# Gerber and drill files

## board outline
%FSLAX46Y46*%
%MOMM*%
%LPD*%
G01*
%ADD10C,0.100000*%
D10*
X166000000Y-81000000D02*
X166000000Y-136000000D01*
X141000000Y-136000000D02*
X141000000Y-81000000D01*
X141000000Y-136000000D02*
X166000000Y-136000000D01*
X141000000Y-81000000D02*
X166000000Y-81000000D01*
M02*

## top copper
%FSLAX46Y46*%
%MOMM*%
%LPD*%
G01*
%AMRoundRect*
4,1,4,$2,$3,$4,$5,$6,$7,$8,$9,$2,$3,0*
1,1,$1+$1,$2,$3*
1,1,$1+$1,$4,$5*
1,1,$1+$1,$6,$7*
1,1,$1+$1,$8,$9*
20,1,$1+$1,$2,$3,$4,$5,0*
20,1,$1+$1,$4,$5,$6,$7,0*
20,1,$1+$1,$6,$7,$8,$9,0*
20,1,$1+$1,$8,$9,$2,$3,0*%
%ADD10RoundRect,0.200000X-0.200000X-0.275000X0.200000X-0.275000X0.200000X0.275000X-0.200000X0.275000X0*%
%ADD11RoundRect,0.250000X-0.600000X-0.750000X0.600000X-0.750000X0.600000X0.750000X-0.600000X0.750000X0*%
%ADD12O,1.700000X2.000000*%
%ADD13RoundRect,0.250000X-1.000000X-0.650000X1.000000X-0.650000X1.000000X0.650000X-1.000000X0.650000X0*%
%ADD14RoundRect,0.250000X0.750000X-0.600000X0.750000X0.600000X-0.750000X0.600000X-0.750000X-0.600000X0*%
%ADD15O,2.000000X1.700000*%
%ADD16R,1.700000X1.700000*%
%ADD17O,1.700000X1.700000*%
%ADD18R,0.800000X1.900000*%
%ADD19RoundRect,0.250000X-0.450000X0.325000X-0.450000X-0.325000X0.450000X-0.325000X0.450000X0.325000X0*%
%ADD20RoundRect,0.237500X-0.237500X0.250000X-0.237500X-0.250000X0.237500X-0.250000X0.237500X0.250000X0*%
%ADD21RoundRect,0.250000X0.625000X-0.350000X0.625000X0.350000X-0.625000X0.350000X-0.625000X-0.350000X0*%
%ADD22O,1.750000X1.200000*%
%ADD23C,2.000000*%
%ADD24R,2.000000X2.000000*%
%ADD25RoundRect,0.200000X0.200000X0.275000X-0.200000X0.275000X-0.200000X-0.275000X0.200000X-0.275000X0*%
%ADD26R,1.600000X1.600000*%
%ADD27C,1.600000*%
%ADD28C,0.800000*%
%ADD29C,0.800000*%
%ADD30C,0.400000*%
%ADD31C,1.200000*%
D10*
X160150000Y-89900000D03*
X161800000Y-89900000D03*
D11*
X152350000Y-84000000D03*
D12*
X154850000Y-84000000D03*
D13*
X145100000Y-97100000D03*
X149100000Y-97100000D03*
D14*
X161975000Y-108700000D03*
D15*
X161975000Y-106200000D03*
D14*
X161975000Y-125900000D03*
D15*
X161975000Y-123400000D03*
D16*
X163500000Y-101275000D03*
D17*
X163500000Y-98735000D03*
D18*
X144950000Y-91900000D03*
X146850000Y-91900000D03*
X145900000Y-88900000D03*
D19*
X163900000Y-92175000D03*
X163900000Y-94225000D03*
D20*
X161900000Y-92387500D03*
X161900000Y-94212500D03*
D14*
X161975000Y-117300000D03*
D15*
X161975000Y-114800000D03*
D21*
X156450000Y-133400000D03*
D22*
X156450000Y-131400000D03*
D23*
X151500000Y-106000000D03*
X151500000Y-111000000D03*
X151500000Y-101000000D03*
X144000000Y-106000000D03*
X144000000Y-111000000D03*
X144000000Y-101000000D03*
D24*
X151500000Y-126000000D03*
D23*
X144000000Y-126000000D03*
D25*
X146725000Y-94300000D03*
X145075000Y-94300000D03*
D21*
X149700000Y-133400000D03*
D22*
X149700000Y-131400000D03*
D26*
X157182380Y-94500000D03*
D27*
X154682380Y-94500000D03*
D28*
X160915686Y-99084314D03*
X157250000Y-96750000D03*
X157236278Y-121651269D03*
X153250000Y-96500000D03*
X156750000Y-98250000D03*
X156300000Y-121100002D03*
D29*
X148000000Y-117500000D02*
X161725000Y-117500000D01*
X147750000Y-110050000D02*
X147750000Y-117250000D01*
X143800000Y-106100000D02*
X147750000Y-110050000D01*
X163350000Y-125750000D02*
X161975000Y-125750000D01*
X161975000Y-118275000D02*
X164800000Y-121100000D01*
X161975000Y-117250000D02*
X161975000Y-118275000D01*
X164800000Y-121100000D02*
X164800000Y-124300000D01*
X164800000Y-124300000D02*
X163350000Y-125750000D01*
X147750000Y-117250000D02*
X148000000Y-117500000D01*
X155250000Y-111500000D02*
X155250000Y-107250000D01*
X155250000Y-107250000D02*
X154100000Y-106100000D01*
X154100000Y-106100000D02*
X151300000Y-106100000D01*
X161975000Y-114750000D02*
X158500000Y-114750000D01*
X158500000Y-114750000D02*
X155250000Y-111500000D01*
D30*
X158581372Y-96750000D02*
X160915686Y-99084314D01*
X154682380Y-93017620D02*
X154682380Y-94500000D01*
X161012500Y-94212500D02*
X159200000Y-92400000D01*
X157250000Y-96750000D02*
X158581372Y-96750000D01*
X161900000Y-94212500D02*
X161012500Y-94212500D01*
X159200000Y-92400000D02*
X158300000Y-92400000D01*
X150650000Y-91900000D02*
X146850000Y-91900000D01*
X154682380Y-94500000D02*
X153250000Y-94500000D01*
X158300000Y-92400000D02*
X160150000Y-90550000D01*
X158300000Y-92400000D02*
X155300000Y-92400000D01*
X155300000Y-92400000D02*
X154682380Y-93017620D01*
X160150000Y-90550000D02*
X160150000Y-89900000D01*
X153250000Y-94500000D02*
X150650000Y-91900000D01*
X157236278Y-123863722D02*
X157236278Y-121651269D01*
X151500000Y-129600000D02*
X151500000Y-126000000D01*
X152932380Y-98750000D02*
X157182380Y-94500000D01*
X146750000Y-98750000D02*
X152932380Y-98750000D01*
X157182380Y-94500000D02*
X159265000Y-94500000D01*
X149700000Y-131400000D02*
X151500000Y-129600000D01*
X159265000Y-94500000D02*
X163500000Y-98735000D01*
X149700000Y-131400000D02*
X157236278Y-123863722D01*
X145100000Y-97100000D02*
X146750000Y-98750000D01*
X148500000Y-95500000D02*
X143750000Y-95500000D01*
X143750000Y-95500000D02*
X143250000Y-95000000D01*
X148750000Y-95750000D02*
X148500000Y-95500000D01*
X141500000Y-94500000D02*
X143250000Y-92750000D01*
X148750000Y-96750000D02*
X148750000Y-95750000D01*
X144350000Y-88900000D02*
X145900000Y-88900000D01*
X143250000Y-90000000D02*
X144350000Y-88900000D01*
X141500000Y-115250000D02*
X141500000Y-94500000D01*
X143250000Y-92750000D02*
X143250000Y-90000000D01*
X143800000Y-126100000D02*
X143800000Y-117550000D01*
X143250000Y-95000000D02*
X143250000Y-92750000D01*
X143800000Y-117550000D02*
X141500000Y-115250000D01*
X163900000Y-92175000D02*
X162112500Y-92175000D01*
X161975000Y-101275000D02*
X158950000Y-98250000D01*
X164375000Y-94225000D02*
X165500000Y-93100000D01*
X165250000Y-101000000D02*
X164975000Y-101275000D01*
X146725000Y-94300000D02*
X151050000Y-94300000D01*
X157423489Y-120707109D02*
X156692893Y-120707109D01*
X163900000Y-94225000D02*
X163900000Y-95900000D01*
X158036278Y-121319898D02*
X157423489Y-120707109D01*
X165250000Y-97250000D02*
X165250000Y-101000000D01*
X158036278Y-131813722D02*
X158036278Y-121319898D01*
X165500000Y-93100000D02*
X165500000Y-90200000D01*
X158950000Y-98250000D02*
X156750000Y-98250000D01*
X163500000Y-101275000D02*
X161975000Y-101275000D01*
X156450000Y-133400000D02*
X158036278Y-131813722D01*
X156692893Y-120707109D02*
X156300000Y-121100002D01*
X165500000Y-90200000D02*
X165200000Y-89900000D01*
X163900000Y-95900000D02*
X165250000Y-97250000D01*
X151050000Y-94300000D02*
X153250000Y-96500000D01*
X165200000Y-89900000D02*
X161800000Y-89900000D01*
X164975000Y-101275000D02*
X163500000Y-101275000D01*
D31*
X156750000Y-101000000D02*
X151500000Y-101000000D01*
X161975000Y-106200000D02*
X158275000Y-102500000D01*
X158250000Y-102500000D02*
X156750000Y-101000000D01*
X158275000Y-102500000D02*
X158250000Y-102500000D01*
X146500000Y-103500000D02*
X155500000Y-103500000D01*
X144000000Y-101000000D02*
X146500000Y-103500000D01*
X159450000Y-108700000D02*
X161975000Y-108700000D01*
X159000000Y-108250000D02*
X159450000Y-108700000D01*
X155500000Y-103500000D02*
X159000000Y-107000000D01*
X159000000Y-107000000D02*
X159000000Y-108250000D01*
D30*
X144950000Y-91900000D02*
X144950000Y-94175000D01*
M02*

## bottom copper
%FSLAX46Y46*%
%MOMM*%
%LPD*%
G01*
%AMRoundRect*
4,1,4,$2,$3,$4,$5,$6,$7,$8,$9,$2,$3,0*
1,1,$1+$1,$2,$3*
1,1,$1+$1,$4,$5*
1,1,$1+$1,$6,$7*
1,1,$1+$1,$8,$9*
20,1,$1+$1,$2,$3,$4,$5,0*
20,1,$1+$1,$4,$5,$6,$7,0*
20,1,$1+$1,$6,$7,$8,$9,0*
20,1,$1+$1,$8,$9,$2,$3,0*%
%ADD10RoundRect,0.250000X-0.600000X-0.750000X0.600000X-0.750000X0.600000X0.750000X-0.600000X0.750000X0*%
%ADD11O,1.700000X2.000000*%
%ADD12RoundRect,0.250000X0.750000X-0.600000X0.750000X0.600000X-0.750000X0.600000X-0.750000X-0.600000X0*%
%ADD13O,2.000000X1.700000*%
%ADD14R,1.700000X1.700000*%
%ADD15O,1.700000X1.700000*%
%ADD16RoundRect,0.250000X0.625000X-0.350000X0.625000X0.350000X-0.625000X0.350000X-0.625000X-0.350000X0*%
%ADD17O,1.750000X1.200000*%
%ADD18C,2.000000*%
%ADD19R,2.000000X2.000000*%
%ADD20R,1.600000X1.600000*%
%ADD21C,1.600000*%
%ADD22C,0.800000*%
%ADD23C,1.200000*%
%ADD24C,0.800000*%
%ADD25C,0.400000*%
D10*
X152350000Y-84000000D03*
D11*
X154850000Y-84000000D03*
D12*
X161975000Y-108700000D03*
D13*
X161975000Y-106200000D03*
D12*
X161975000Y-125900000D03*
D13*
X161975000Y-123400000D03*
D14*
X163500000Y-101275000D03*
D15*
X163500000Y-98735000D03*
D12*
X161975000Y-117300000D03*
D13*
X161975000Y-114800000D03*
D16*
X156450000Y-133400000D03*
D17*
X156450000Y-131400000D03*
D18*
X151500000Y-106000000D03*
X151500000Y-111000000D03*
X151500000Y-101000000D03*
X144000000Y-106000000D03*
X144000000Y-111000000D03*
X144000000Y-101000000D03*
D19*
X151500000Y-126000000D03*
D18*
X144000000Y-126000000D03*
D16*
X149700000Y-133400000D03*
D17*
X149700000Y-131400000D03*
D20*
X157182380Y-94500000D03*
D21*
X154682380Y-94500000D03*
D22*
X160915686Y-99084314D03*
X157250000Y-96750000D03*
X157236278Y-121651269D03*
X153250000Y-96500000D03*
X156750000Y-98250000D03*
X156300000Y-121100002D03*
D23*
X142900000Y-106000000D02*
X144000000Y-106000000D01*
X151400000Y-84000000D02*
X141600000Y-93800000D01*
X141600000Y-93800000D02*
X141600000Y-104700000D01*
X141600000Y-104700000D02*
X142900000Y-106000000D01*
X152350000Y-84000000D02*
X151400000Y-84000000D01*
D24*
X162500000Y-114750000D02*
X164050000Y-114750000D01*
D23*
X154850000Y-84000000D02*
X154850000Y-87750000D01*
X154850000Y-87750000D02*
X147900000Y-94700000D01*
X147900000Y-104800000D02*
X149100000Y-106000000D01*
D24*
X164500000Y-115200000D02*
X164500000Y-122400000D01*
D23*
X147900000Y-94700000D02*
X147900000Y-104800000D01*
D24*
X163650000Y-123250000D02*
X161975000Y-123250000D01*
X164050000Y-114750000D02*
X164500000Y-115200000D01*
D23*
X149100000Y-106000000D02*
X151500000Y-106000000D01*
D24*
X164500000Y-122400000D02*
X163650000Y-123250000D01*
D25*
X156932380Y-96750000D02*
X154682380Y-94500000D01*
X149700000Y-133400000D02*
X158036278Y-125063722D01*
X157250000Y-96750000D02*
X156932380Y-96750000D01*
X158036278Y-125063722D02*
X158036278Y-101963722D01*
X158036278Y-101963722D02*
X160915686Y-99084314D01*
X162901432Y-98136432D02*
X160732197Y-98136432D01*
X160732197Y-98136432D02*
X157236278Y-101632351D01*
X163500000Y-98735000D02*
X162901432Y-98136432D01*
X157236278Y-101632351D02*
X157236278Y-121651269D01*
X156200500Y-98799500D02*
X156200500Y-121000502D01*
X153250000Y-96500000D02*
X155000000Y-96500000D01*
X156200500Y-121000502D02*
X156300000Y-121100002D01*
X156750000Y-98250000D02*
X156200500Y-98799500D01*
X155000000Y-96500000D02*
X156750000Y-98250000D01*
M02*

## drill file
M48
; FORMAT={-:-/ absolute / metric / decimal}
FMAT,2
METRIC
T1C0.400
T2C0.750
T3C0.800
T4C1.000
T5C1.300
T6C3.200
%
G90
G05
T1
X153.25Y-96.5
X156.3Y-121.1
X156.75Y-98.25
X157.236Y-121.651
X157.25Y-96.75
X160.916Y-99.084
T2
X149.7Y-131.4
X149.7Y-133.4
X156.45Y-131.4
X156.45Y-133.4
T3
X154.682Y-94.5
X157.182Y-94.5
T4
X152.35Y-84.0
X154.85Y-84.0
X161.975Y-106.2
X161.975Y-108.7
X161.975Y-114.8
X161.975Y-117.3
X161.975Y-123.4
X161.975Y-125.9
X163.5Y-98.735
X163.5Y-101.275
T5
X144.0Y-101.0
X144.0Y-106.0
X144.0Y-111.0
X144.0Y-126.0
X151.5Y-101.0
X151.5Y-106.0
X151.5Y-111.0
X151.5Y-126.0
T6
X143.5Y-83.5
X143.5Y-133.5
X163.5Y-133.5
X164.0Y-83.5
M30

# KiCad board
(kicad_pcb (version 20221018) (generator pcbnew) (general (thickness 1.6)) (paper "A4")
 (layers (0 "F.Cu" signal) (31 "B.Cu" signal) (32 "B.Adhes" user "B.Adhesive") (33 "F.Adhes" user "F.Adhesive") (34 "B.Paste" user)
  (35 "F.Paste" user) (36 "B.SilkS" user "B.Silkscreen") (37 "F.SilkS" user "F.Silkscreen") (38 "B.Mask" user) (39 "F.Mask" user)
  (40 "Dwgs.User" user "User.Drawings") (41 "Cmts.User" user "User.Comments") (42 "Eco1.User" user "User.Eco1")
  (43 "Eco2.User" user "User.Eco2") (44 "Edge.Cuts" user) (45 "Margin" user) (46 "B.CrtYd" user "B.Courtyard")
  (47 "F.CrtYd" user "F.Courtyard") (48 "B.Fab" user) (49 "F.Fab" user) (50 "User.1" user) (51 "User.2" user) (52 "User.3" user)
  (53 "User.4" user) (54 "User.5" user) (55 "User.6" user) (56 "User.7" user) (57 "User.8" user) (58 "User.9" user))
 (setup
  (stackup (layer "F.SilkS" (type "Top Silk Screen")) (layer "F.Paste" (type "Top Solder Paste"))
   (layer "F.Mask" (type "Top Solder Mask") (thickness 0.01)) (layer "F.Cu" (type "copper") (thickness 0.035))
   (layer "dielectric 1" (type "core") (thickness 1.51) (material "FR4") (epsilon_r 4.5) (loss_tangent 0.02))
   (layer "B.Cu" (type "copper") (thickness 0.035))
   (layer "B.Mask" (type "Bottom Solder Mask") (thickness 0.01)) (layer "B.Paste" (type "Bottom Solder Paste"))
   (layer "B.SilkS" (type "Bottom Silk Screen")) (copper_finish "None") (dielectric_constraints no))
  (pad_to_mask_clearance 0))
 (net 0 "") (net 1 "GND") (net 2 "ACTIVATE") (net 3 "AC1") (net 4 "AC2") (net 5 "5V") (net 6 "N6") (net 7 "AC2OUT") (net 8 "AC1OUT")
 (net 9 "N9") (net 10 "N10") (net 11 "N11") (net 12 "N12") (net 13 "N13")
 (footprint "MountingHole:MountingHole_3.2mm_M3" (layer "F.Cu") (at 163.5 133.5)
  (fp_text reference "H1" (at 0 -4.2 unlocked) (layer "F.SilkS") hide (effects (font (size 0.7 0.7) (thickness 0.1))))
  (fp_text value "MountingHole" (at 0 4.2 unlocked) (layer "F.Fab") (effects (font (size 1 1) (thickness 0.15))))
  (pad "" np_thru_hole circle (at 0 0) (size 3.2 3.2) (drill 3.2) (layers "*.Cu" "*.Mask")))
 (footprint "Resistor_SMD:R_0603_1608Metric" (layer "F.Cu") (at 160.975 89.9)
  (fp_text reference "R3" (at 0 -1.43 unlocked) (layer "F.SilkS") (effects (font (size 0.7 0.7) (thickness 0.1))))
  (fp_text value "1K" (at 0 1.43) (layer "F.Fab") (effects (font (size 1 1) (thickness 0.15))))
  (pad "1" smd roundrect (at -0.825 0) (size 0.8 0.95) (layers "F.Cu" "F.Paste" "F.Mask") (roundrect_rratio 0.25) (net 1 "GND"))
  (pad "2" smd roundrect (at 0.825 0) (size 0.8 0.95) (layers "F.Cu" "F.Paste" "F.Mask") (roundrect_rratio 0.25) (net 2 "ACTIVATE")))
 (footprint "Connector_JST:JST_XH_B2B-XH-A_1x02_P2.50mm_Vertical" (layer "F.Cu") (at 152.35 84)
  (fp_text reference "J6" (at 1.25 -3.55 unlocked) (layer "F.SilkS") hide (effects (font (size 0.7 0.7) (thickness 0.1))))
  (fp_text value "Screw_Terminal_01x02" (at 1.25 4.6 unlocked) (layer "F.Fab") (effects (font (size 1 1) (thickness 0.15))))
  (pad "1" thru_hole roundrect (at 0 0) (size 1.7 2) (drill 1) (layers "*.Cu" "*.Mask") (roundrect_rratio 0.1470588235) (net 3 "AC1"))
  (pad "2" thru_hole oval (at 2.5 0) (size 1.7 2) (drill 1) (layers "*.Cu" "*.Mask") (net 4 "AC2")))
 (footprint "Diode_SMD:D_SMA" (layer "F.Cu") (at 147.1 97.1)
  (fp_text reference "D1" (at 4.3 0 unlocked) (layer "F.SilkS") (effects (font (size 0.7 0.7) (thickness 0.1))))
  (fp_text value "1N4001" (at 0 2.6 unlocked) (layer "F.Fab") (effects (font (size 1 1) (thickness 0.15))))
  (pad "1" smd roundrect (at -2 0) (size 2.5 1.8) (layers "F.Cu" "F.Paste" "F.Mask") (roundrect_rratio 0.1388888889) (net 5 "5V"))
  (pad "2" smd roundrect (at 2 0) (size 2.5 1.8) (layers "F.Cu" "F.Paste" "F.Mask") (roundrect_rratio 0.1388888889) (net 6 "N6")))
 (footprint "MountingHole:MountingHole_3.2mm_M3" (layer "F.Cu") (at 164 83.5)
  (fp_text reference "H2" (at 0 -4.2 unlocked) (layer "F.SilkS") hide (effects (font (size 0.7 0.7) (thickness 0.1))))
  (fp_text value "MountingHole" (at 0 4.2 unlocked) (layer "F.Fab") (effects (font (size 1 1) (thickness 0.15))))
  (pad "" np_thru_hole circle (at 0 0) (size 3.2 3.2) (drill 3.2) (layers "*.Cu" "*.Mask")))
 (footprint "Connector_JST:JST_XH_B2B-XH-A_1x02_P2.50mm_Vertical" (layer "F.Cu") (at 161.975 108.7 90)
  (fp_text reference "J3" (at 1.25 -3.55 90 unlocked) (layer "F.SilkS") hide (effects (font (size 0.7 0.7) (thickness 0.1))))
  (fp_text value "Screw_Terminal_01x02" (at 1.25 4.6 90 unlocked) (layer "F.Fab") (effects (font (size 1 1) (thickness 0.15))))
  (pad "1" thru_hole roundrect (at 0 0 90) (size 1.7 2) (drill 1) (layers "*.Cu" "*.Mask") (roundrect_rratio 0.1470588235) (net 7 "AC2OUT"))
  (pad "2" thru_hole oval (at 2.5 0 90) (size 1.7 2) (drill 1) (layers "*.Cu" "*.Mask") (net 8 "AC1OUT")))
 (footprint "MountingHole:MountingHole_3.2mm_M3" (layer "F.Cu") (at 143.5 83.5)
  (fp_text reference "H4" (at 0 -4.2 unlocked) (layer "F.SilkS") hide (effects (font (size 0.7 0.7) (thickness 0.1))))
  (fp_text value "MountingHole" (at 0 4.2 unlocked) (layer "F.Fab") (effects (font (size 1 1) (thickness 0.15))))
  (pad "" np_thru_hole circle (at 0 0) (size 3.2 3.2) (drill 3.2) (layers "*.Cu" "*.Mask")))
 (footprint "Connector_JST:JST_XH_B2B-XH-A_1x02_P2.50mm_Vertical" (layer "F.Cu") (at 161.975 125.9 90)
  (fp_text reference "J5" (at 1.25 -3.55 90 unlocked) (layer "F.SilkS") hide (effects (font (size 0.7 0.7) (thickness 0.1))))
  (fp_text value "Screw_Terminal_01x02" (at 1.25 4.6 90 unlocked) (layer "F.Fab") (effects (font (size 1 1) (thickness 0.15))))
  (pad "1" thru_hole roundrect (at 0 0 90) (size 1.7 2) (drill 1) (layers "*.Cu" "*.Mask") (roundrect_rratio 0.1470588235) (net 3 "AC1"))
  (pad "2" thru_hole oval (at 2.5 0 90) (size 1.7 2) (drill 1) (layers "*.Cu" "*.Mask") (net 4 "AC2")))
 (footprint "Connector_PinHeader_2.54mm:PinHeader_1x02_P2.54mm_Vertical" (layer "F.Cu") (at 163.5 101.275 180)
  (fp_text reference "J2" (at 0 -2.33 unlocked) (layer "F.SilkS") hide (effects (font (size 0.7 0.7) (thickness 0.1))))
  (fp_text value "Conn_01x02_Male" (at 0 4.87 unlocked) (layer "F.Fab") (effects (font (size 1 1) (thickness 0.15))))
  (pad "1" thru_hole rect (at 0 0 180) (size 1.7 1.7) (drill 1) (layers "*.Cu" "*.Mask") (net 2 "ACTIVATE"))
  (pad "2" thru_hole oval (at 0 2.54 180) (size 1.7 1.7) (drill 1) (layers "*.Cu" "*.Mask") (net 5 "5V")))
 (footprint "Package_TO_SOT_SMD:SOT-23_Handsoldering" (layer "F.Cu") (at 145.9 90.4 90)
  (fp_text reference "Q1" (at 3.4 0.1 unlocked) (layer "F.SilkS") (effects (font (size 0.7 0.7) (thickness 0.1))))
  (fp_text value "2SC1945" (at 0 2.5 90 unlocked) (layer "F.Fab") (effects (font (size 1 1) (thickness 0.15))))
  (pad "1" smd rect (at -1.5 -0.95 90) (size 1.9 0.8) (layers "F.Cu" "F.Paste" "F.Mask") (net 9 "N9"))
  (pad "2" smd rect (at -1.5 0.95 90) (size 1.9 0.8) (layers "F.Cu" "F.Paste" "F.Mask") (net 1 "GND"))
  (pad "3" smd rect (at 1.5 0 90) (size 1.9 0.8) (layers "F.Cu" "F.Paste" "F.Mask") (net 6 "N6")))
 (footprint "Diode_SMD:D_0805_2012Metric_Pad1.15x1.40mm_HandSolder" (layer "F.Cu") (at 163.9 93.2 -90)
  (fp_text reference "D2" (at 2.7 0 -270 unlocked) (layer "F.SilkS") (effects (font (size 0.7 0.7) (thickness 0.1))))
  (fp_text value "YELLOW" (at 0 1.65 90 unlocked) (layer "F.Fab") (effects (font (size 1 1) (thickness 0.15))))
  (pad "1" smd roundrect (at -1.025 0 270) (size 1.15 1.4) (layers "F.Cu" "F.Paste" "F.Mask") (roundrect_rratio 0.2173913043) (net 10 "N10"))
  (pad "2" smd roundrect (at 1.025 0 270) (size 1.15 1.4) (layers "F.Cu" "F.Paste" "F.Mask") (roundrect_rratio 0.2173913043)
   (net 2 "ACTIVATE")))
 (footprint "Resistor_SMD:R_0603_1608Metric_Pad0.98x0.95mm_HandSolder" (layer "F.Cu") (at 161.9 93.3 -90)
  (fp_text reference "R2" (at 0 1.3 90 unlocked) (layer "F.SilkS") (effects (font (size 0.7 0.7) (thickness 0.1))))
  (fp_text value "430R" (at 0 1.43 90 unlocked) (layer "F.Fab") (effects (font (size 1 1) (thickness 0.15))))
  (pad "1" smd roundrect (at -0.9125 0 270) (size 0.975 0.95) (layers "F.Cu" "F.Paste" "F.Mask") (roundrect_rratio 0.25) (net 10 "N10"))
  (pad "2" smd roundrect (at 0.9125 0 270) (size 0.975 0.95) (layers "F.Cu" "F.Paste" "F.Mask") (roundrect_rratio 0.25) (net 1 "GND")))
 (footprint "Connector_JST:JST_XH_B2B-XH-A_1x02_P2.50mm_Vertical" (layer "F.Cu") (at 161.975 117.3 90)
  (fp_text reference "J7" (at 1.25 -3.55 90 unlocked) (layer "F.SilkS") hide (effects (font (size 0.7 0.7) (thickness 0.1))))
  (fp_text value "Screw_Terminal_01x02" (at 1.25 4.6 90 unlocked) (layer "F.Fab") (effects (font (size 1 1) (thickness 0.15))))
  (pad "1" thru_hole roundrect (at 0 0 90) (size 1.7 2) (drill 1) (layers "*.Cu" "*.Mask") (roundrect_rratio 0.1470588235) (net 3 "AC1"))
  (pad "2" thru_hole oval (at 2.5 0 90) (size 1.7 2) (drill 1) (layers "*.Cu" "*.Mask") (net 4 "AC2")))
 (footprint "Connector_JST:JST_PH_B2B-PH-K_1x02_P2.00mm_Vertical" (layer "F.Cu") (at 156.45 133.4 90)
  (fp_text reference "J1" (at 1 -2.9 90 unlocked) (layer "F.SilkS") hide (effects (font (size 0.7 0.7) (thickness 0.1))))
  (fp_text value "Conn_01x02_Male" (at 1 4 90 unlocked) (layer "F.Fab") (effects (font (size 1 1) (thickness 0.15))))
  (pad "1" thru_hole roundrect (at 0 0 90) (size 1.2 1.75) (drill 0.75) (layers "*.Cu" "*.Mask") (roundrect_rratio 0.2083333333)
   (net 2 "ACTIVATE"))
  (pad "2" thru_hole oval (at 2 0 90) (size 1.2 1.75) (drill 0.75) (layers "*.Cu" "*.Mask") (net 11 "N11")))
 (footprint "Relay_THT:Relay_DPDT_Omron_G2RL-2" (layer "F.Cu") (at 151.5 126 180)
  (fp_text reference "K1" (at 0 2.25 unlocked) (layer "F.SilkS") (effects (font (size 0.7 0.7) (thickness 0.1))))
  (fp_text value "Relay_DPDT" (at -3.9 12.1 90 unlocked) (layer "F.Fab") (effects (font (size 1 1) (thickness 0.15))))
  (pad "11" thru_hole circle (at 0 20 180) (size 2 2) (drill 1.3) (layers "*.Cu" "*.Mask") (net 4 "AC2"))
  (pad "12" thru_hole circle (at 0 15 180) (size 2 2) (drill 1.3) (layers "*.Cu" "*.Mask") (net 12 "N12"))
  (pad "14" thru_hole circle (at 0 25 180) (size 2 2) (drill 1.3) (layers "*.Cu" "*.Mask") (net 8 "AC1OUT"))
  (pad "21" thru_hole circle (at 7.5 20 180) (size 2 2) (drill 1.3) (layers "*.Cu" "*.Mask") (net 3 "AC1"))
  (pad "22" thru_hole circle (at 7.5 15 180) (size 2 2) (drill 1.3) (layers "*.Cu" "*.Mask") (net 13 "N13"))
  (pad "24" thru_hole circle (at 7.5 25 180) (size 2 2) (drill 1.3) (layers "*.Cu" "*.Mask") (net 7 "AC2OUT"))
  (pad "A1" thru_hole rect (at 0 0 180) (size 2 2) (drill 1.3) (layers "*.Cu" "*.Mask") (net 5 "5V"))
  (pad "A2" thru_hole circle (at 7.5 0 180) (size 2 2) (drill 1.3) (layers "*.Cu" "*.Mask") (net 6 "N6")))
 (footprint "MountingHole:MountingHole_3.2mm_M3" (layer "F.Cu") (at 143.5 133.5)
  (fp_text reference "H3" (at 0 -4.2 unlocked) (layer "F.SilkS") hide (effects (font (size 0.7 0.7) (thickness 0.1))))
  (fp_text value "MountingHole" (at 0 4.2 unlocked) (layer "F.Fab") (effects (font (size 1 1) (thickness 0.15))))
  (pad "" np_thru_hole circle (at 0 0) (size 3.2 3.2) (drill 3.2) (layers "*.Cu" "*.Mask")))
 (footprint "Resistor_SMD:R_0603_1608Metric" (layer "F.Cu") (at 145.9 94.3 180)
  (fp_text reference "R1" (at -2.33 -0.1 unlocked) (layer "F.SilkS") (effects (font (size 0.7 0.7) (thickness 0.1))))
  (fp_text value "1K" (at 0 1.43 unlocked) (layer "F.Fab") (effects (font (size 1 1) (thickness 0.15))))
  (pad "1" smd roundrect (at -0.825 0 180) (size 0.8 0.95) (layers "F.Cu" "F.Paste" "F.Mask") (roundrect_rratio 0.25) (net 2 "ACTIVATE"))
  (pad "2" smd roundrect (at 0.825 0 180) (size 0.8 0.95) (layers "F.Cu" "F.Paste" "F.Mask") (roundrect_rratio 0.25) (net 9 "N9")))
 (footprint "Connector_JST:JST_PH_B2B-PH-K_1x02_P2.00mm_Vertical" (layer "F.Cu") (at 149.7 133.4 90)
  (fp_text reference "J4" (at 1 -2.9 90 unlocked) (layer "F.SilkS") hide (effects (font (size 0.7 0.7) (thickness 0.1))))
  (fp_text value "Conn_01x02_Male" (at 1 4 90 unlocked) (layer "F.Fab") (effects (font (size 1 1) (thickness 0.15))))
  (pad "1" thru_hole roundrect (at 0 0 90) (size 1.2 1.75) (drill 0.75) (layers "*.Cu" "*.Mask") (roundrect_rratio 0.2083333333)
   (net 1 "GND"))
  (pad "2" thru_hole oval (at 2 0 90) (size 1.2 1.75) (drill 0.75) (layers "*.Cu" "*.Mask") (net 5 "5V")))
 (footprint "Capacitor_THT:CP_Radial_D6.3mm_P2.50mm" (layer "F.Cu") (at 157.18238 94.5 180)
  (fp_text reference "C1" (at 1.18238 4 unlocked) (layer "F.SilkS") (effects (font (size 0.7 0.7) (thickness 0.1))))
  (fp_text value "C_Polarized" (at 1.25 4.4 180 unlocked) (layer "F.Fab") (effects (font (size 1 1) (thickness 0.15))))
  (pad "1" thru_hole rect (at 0 0 180) (size 1.6 1.6) (drill 0.8) (layers "*.Cu" "*.Mask") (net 5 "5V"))
  (pad "2" thru_hole circle (at 2.5 0 180) (size 1.6 1.6) (drill 0.8) (layers "*.Cu" "*.Mask") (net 1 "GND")))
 (gr_line (start 166 81) (end 166 136) (stroke (width 0.1) (type solid)) (layer "Edge.Cuts"))
 (gr_line (start 141 136) (end 141 81) (stroke (width 0.1) (type solid)) (layer "Edge.Cuts"))
 (gr_line (start 141 136) (end 166 136) (stroke (width 0.1) (type solid)) (layer "Edge.Cuts"))
 (gr_line (start 141 81) (end 166 81) (stroke (width 0.1) (type solid)) (layer "Edge.Cuts"))
 (segment (start 148 117.5) (end 161.725 117.5) (width 0.8) (layer "F.Cu") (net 3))
 (segment (start 147.75 110.05) (end 147.75 117.25) (width 0.8) (layer "F.Cu") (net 3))
 (segment (start 143.8 106.1) (end 147.75 110.05) (width 0.8) (layer "F.Cu") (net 3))
 (segment (start 163.35 125.75) (end 161.975 125.75) (width 0.8) (layer "F.Cu") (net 3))
 (segment (start 161.975 118.275) (end 164.8 121.1) (width 0.8) (layer "F.Cu") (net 3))
 (segment (start 161.975 117.25) (end 161.975 118.275) (width 0.8) (layer "F.Cu") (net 3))
 (segment (start 164.8 121.1) (end 164.8 124.3) (width 0.8) (layer "F.Cu") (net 3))
 (segment (start 164.8 124.3) (end 163.35 125.75) (width 0.8) (layer "F.Cu") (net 3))
 (segment (start 147.75 117.25) (end 148 117.5) (width 0.8) (layer "F.Cu") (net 3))
 (segment (start 142.9 106) (end 144 106) (width 1.2) (layer "B.Cu") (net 3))
 (segment (start 151.4 84) (end 141.6 93.8) (width 1.2) (layer "B.Cu") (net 3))
 (segment (start 141.6 93.8) (end 141.6 104.7) (width 1.2) (layer "B.Cu") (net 3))
 (segment (start 141.6 104.7) (end 142.9 106) (width 1.2) (layer "B.Cu") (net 3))
 (segment (start 152.35 84) (end 151.4 84) (width 1.2) (layer "B.Cu") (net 3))
 (segment (start 155.25 111.5) (end 155.25 107.25) (width 0.8) (layer "F.Cu") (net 4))
 (segment (start 155.25 107.25) (end 154.1 106.1) (width 0.8) (layer "F.Cu") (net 4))
 (segment (start 154.1 106.1) (end 151.3 106.1) (width 0.8) (layer "F.Cu") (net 4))
 (segment (start 161.975 114.75) (end 158.5 114.75) (width 0.8) (layer "F.Cu") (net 4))
 (segment (start 158.5 114.75) (end 155.25 111.5) (width 0.8) (layer "F.Cu") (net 4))
 (segment (start 162.5 114.75) (end 164.05 114.75) (width 0.8) (layer "B.Cu") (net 4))
 (segment (start 154.85 84) (end 154.85 87.75) (width 1.2) (layer "B.Cu") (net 4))
 (segment (start 154.85 87.75) (end 147.9 94.7) (width 1.2) (layer "B.Cu") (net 4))
 (segment (start 147.9 104.8) (end 149.1 106) (width 1.2) (layer "B.Cu") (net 4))
 (segment (start 164.5 115.2) (end 164.5 122.4) (width 0.8) (layer "B.Cu") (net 4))
 (segment (start 147.9 94.7) (end 147.9 104.8) (width 1.2) (layer "B.Cu") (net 4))
 (segment (start 163.65 123.25) (end 161.975 123.25) (width 0.8) (layer "B.Cu") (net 4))
 (segment (start 164.05 114.75) (end 164.5 115.2) (width 0.8) (layer "B.Cu") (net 4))
 (segment (start 149.1 106) (end 151.5 106) (width 1.2) (layer "B.Cu") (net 4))
 (segment (start 164.5 122.4) (end 163.65 123.25) (width 0.8) (layer "B.Cu") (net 4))
 (segment (start 158.581372 96.75) (end 160.915686 99.084314) (width 0.4) (layer "F.Cu") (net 1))
 (segment (start 154.68238 93.01762) (end 154.68238 94.5) (width 0.4) (layer "F.Cu") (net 1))
 (segment (start 161.0125 94.2125) (end 159.2 92.4) (width 0.4) (layer "F.Cu") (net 1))
 (segment (start 157.25 96.75) (end 158.581372 96.75) (width 0.4) (layer "F.Cu") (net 1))
 (segment (start 161.9 94.2125) (end 161.0125 94.2125) (width 0.4) (layer "F.Cu") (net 1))
 (segment (start 159.2 92.4) (end 158.3 92.4) (width 0.4) (layer "F.Cu") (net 1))
 (segment (start 150.65 91.9) (end 146.85 91.9) (width 0.4) (layer "F.Cu") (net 1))
 (segment (start 154.68238 94.5) (end 153.25 94.5) (width 0.4) (layer "F.Cu") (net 1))
 (segment (start 158.3 92.4) (end 160.15 90.55) (width 0.4) (layer "F.Cu") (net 1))
 (segment (start 158.3 92.4) (end 155.3 92.4) (width 0.4) (layer "F.Cu") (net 1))
 (segment (start 155.3 92.4) (end 154.68238 93.01762) (width 0.4) (layer "F.Cu") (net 1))
 (segment (start 160.15 90.55) (end 160.15 89.9) (width 0.4) (layer "F.Cu") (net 1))
 (segment (start 153.25 94.5) (end 150.65 91.9) (width 0.4) (layer "F.Cu") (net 1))
 (via (at 160.915686 99.084314) (size 0.8) (drill 0.4) (layers "F.Cu" "B.Cu") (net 1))
 (via (at 157.25 96.75) (size 0.8) (drill 0.4) (layers "F.Cu" "B.Cu") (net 1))
 (segment (start 156.93238 96.75) (end 154.68238 94.5) (width 0.4) (layer "B.Cu") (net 1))
 (segment (start 149.7 133.4) (end 158.036278 125.063722) (width 0.4) (layer "B.Cu") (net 1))
 (segment (start 157.25 96.75) (end 156.93238 96.75) (width 0.4) (layer "B.Cu") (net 1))
 (segment (start 158.036278 125.063722) (end 158.036278 101.963722) (width 0.4) (layer "B.Cu") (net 1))
 (segment (start 158.036278 101.963722) (end 160.915686 99.084314) (width 0.4) (layer "B.Cu") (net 1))
 (segment (start 157.236278 123.863722) (end 157.236278 121.651269) (width 0.4) (layer "F.Cu") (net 5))
 (segment (start 151.5 129.6) (end 151.5 126) (width 0.4) (layer "F.Cu") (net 5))
 (segment (start 152.93238 98.75) (end 157.18238 94.5) (width 0.4) (layer "F.Cu") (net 5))
 (segment (start 146.75 98.75) (end 152.93238 98.75) (width 0.4) (layer "F.Cu") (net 5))
 (segment (start 157.18238 94.5) (end 159.265 94.5) (width 0.4) (layer "F.Cu") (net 5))
 (segment (start 149.7 131.4) (end 151.5 129.6) (width 0.4) (layer "F.Cu") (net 5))
 (segment (start 159.265 94.5) (end 163.5 98.735) (width 0.4) (layer "F.Cu") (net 5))
 (segment (start 149.7 131.4) (end 157.236278 123.863722) (width 0.4) (layer "F.Cu") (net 5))
 (segment (start 145.1 97.1) (end 146.75 98.75) (width 0.4) (layer "F.Cu") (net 5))
 (via (at 157.236278 121.651269) (size 0.8) (drill 0.4) (layers "F.Cu" "B.Cu") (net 5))
 (segment (start 162.901432 98.136432) (end 160.732197 98.136432) (width 0.4) (layer "B.Cu") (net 5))
 (segment (start 160.732197 98.136432) (end 157.236278 101.632351) (width 0.4) (layer "B.Cu") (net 5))
 (segment (start 163.5 98.735) (end 162.901432 98.136432) (width 0.4) (layer "B.Cu") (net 5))
 (segment (start 157.236278 101.632351) (end 157.236278 121.651269) (width 0.4) (layer "B.Cu") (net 5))
 (segment (start 148.5 95.5) (end 143.75 95.5) (width 0.4) (layer "F.Cu") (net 6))
 (segment (start 143.75 95.5) (end 143.25 95) (width 0.4) (layer "F.Cu") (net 6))
 (segment (start 148.75 95.75) (end 148.5 95.5) (width 0.4) (layer "F.Cu") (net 6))
 (segment (start 141.5 94.5) (end 143.25 92.75) (width 0.4) (layer "F.Cu") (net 6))
 (segment (start 148.75 96.75) (end 148.75 95.75) (width 0.4) (layer "F.Cu") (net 6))
 (segment (start 144.35 88.9) (end 145.9 88.9) (width 0.4) (layer "F.Cu") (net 6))
 (segment (start 143.25 90) (end 144.35 88.9) (width 0.4) (layer "F.Cu") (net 6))
 (segment (start 141.5 115.25) (end 141.5 94.5) (width 0.4) (layer "F.Cu") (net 6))
 (segment (start 143.25 92.75) (end 143.25 90) (width 0.4) (layer "F.Cu") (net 6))
 (segment (start 143.8 126.1) (end 143.8 117.55) (width 0.4) (layer "F.Cu") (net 6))
 (segment (start 143.25 95) (end 143.25 92.75) (width 0.4) (layer "F.Cu") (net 6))
 (segment (start 143.8 117.55) (end 141.5 115.25) (width 0.4) (layer "F.Cu") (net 6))
 (segment (start 163.9 92.175) (end 162.1125 92.175) (width 0.4) (layer "F.Cu") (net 10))
 (segment (start 161.975 101.275) (end 158.95 98.25) (width 0.4) (layer "F.Cu") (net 2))
 (segment (start 164.375 94.225) (end 165.5 93.1) (width 0.4) (layer "F.Cu") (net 2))
 (segment (start 165.25 101) (end 164.975 101.275) (width 0.4) (layer "F.Cu") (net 2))
 (segment (start 146.725 94.3) (end 151.05 94.3) (width 0.4) (layer "F.Cu") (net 2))
 (segment (start 157.423489 120.707109) (end 156.692893 120.707109) (width 0.4) (layer "F.Cu") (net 2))
 (segment (start 163.9 94.225) (end 163.9 95.9) (width 0.4) (layer "F.Cu") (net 2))
 (segment (start 158.036278 121.319898) (end 157.423489 120.707109) (width 0.4) (layer "F.Cu") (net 2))
 (segment (start 165.25 97.25) (end 165.25 101) (width 0.4) (layer "F.Cu") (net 2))
 (segment (start 158.036278 131.813722) (end 158.036278 121.319898) (width 0.4) (layer "F.Cu") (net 2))
 (segment (start 165.5 93.1) (end 165.5 90.2) (width 0.4) (layer "F.Cu") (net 2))
 (segment (start 158.95 98.25) (end 156.75 98.25) (width 0.4) (layer "F.Cu") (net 2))
 (segment (start 163.5 101.275) (end 161.975 101.275) (width 0.4) (layer "F.Cu") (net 2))
 (segment (start 156.45 133.4) (end 158.036278 131.813722) (width 0.4) (layer "F.Cu") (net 2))
 (segment (start 156.692893 120.707109) (end 156.3 121.100002) (width 0.4) (layer "F.Cu") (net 2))
 (segment (start 165.5 90.2) (end 165.2 89.9) (width 0.4) (layer "F.Cu") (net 2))
 (segment (start 163.9 95.9) (end 165.25 97.25) (width 0.4) (layer "F.Cu") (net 2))
 (segment (start 151.05 94.3) (end 153.25 96.5) (width 0.4) (layer "F.Cu") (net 2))
 (segment (start 165.2 89.9) (end 161.8 89.9) (width 0.4) (layer "F.Cu") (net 2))
 (segment (start 164.975 101.275) (end 163.5 101.275) (width 0.4) (layer "F.Cu") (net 2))
 (via (at 153.25 96.5) (size 0.8) (drill 0.4) (layers "F.Cu" "B.Cu") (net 2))
 (via (at 156.75 98.25) (size 0.8) (drill 0.4) (layers "F.Cu" "B.Cu") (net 2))
 (via (at 156.3 121.100002) (size 0.8) (drill 0.4) (layers "F.Cu" "B.Cu") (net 2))
 (segment (start 156.2005 98.7995) (end 156.2005 121.000502) (width 0.4) (layer "B.Cu") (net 2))
 (segment (start 153.25 96.5) (end 155 96.5) (width 0.4) (layer "B.Cu") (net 2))
 (segment (start 156.2005 121.000502) (end 156.3 121.100002) (width 0.4) (layer "B.Cu") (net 2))
 (segment (start 156.75 98.25) (end 156.2005 98.7995) (width 0.4) (layer "B.Cu") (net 2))
 (segment (start 155 96.5) (end 156.75 98.25) (width 0.4) (layer "B.Cu") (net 2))
 (segment (start 156.75 101) (end 151.5 101) (width 1.2) (layer "F.Cu") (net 8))
 (segment (start 161.975 106.2) (end 158.275 102.5) (width 1.2) (layer "F.Cu") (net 8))
 (segment (start 158.25 102.5) (end 156.75 101) (width 1.2) (layer "F.Cu") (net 8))
 (segment (start 158.275 102.5) (end 158.25 102.5) (width 1.2) (layer "F.Cu") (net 8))
 (segment (start 146.5 103.5) (end 155.5 103.5) (width 1.2) (layer "F.Cu") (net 7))
 (segment (start 144 101) (end 146.5 103.5) (width 1.2) (layer "F.Cu") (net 7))
 (segment (start 159.45 108.7) (end 161.975 108.7) (width 1.2) (layer "F.Cu") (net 7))
 (segment (start 159 108.25) (end 159.45 108.7) (width 1.2) (layer "F.Cu") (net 7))
 (segment (start 155.5 103.5) (end 159 107) (width 1.2) (layer "F.Cu") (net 7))
 (segment (start 159 107) (end 159 108.25) (width 1.2) (layer "F.Cu") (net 7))
 (segment (start 144.95 91.9) (end 144.95 94.175) (width 0.4) (layer "F.Cu") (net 9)))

